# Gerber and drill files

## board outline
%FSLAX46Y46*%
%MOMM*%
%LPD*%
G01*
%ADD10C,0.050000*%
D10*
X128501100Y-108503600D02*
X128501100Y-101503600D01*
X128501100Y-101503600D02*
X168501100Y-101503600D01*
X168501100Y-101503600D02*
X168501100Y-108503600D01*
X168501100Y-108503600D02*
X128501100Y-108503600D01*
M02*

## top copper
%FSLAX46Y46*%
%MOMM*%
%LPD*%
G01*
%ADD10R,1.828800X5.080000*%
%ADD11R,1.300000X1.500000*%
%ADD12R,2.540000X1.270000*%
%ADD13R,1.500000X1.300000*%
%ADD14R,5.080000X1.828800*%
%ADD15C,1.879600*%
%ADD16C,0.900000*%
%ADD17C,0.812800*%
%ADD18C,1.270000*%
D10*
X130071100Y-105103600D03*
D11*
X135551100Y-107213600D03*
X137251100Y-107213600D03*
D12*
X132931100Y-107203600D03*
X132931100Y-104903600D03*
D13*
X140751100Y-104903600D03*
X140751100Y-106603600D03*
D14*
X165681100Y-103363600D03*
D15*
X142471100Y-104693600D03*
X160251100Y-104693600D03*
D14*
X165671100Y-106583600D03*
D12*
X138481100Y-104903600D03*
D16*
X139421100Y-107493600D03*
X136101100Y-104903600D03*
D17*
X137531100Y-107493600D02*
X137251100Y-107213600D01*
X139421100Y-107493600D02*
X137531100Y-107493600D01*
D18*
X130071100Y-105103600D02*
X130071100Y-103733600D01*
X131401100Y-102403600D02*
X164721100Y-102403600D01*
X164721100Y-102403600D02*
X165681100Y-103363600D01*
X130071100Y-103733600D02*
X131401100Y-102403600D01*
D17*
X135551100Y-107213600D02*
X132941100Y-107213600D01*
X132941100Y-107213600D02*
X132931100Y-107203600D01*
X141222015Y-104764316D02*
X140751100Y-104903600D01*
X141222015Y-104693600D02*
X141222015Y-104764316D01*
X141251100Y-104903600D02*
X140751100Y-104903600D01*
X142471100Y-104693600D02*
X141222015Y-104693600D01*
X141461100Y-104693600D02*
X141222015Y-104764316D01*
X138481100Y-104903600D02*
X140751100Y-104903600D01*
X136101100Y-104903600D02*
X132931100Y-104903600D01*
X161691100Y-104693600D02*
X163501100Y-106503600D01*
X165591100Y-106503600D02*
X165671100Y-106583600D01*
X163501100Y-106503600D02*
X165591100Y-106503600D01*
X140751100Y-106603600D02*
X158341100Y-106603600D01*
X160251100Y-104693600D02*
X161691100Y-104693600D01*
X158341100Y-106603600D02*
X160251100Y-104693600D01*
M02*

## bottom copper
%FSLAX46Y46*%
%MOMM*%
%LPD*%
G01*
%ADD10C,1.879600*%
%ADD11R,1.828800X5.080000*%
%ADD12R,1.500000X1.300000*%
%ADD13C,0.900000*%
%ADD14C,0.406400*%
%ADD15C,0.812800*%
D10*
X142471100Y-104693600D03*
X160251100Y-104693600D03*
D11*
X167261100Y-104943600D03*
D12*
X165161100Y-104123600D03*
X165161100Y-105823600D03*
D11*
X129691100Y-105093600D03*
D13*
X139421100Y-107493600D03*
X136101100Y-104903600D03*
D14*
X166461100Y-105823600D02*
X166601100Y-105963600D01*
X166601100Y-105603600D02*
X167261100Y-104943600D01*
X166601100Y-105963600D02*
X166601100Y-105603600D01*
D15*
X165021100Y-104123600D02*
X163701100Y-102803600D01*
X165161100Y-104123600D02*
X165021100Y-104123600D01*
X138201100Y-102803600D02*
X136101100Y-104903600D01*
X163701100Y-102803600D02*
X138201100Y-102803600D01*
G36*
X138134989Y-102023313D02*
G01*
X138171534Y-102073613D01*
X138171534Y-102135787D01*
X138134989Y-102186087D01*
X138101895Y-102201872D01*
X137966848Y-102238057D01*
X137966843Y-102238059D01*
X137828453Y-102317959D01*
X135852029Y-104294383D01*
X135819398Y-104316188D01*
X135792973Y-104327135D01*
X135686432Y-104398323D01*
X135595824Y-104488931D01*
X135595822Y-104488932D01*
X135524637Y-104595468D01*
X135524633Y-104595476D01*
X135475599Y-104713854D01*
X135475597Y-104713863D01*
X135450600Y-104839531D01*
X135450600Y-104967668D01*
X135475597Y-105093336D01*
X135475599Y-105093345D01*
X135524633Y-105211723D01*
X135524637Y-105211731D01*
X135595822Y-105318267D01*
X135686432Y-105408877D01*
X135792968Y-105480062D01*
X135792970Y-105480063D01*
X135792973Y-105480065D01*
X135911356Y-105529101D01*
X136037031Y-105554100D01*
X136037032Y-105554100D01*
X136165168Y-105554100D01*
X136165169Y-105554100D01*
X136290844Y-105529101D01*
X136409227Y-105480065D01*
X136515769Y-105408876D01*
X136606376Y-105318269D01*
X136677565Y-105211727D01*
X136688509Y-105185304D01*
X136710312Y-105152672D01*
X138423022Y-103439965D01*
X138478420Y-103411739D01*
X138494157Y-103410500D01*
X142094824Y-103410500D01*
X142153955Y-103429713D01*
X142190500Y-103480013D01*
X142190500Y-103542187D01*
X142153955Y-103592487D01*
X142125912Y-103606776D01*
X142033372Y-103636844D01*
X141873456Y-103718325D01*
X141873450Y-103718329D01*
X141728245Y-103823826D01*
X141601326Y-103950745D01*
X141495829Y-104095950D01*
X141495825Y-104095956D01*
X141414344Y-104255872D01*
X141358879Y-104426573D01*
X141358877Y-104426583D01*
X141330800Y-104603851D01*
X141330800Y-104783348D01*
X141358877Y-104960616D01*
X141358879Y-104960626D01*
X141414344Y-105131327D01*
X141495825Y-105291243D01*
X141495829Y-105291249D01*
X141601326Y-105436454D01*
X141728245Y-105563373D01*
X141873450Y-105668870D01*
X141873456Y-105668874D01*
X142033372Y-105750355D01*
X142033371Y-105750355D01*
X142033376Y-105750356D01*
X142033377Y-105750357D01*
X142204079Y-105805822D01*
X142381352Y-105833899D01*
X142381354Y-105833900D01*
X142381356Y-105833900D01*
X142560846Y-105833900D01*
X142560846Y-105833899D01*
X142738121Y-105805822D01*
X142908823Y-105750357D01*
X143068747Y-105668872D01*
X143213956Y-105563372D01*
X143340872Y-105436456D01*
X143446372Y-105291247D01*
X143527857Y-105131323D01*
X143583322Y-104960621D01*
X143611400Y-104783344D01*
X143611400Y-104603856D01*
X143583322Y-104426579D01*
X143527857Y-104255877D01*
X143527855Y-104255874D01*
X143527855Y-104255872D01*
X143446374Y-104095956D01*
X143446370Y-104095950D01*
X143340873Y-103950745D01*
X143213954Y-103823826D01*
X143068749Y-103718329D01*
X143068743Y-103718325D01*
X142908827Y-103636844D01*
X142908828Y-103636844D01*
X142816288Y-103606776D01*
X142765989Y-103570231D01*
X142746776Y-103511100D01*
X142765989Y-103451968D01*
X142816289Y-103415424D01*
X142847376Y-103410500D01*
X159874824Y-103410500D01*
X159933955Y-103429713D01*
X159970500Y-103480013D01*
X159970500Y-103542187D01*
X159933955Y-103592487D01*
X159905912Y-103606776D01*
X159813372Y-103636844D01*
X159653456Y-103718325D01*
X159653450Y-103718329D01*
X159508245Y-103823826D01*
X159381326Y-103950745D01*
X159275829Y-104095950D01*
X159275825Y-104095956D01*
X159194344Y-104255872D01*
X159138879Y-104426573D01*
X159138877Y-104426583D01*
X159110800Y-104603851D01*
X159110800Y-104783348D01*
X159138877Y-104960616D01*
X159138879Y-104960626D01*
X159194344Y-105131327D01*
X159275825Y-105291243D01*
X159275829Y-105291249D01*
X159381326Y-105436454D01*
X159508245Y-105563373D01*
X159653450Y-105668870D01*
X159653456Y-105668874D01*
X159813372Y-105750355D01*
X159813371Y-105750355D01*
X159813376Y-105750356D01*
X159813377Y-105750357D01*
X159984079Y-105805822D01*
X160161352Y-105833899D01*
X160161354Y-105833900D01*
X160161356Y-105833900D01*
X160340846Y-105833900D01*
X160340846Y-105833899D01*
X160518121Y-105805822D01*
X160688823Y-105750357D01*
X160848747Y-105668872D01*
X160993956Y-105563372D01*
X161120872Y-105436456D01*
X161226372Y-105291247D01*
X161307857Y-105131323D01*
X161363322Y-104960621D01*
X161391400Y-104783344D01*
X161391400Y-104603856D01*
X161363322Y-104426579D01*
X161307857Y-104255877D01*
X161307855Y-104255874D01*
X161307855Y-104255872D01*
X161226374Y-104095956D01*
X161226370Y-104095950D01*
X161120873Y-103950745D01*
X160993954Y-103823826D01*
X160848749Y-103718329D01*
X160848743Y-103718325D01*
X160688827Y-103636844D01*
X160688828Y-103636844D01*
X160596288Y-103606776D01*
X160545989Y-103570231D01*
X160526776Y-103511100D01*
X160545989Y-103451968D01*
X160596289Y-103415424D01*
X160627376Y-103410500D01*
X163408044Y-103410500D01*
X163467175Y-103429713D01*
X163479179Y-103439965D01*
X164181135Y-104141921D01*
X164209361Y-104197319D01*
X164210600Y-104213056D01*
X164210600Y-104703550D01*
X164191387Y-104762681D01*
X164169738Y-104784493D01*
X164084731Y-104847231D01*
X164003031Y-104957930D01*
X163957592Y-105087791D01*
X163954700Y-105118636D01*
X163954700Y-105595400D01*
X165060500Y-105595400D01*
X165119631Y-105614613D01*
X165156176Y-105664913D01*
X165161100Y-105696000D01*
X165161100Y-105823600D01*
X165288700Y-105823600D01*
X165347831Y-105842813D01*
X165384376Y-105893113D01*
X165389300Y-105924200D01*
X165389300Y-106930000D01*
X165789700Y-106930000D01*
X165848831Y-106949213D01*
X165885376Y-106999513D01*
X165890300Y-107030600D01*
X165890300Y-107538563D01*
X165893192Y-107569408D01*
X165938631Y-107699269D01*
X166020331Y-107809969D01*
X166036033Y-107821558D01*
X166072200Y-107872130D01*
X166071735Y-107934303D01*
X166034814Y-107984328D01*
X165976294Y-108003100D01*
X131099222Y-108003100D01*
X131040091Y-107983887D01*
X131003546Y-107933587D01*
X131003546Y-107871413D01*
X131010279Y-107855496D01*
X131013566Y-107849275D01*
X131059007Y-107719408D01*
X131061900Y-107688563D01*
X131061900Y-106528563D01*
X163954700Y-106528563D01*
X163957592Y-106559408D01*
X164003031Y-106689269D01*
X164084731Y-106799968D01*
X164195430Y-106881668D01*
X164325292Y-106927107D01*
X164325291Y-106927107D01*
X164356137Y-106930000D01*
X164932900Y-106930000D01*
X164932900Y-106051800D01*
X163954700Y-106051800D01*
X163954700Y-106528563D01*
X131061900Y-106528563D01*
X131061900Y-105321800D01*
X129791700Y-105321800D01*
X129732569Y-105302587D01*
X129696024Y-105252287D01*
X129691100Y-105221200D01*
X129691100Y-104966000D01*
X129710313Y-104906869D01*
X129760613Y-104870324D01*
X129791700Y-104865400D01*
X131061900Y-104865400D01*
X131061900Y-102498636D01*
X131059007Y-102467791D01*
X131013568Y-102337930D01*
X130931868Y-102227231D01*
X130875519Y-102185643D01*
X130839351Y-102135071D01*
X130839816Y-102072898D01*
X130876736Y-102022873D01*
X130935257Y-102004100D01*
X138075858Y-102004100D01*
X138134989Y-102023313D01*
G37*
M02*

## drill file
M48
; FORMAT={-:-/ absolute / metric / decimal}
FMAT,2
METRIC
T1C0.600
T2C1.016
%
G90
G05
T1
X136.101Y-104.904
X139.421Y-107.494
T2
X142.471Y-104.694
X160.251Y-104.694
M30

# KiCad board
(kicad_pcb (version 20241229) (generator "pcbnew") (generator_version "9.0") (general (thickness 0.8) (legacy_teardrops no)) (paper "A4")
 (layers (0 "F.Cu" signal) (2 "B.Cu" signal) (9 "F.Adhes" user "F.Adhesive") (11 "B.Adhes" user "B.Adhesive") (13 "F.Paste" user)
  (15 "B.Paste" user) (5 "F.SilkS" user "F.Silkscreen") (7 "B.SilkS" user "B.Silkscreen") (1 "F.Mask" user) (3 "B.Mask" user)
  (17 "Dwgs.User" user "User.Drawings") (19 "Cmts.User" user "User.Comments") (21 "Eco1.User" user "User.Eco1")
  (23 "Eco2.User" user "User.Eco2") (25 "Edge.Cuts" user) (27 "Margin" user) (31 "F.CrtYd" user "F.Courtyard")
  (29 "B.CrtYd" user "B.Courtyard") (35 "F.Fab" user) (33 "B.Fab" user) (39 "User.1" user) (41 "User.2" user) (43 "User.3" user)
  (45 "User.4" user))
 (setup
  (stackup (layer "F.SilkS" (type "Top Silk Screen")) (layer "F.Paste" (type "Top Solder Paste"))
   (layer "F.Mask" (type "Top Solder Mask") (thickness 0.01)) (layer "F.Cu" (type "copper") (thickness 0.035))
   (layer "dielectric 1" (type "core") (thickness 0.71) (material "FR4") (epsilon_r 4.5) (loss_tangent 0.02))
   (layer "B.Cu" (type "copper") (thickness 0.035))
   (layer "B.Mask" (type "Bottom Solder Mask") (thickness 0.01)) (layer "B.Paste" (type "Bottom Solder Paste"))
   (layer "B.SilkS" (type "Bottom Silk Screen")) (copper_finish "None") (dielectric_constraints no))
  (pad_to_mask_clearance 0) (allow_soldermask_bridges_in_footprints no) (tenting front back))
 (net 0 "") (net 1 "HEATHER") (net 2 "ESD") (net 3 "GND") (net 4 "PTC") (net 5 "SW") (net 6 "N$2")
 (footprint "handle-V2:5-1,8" (layer "F.Cu") (at 130.0711 105.1036 180)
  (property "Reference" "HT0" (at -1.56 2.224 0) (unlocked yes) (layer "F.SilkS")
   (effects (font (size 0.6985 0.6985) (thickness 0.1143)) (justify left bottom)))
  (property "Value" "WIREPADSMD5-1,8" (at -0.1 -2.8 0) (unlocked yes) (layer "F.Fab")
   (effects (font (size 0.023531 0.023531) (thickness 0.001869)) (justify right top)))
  (pad "1" smd rect (at 0 0 180) (size 1.8288 5.08) (layers "F.Cu" "F.Mask" "F.Paste") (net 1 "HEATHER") (solder_mask_margin 0)
   (solder_paste_margin 0) (thermal_bridge_angle 0)))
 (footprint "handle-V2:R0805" (layer "F.Cu") (at 136.4011 107.2136)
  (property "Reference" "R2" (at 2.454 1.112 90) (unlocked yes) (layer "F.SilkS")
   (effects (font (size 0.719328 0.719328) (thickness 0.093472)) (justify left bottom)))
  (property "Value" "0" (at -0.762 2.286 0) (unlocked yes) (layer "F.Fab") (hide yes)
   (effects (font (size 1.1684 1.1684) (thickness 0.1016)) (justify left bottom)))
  (pad "1" smd rect (at -0.85 0) (size 1.3 1.5) (layers "F.Cu" "F.Mask" "F.Paste") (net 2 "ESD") (solder_mask_margin 0)
   (solder_paste_margin 0) (thermal_bridge_angle 0))
  (pad "2" smd rect (at 0.85 0) (size 1.3 1.5) (layers "F.Cu" "F.Mask" "F.Paste") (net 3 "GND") (solder_mask_margin 0)
   (solder_paste_margin 0) (thermal_bridge_angle 0)))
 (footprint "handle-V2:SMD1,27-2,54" (layer "F.Cu") (at 132.9311 107.2036 -90)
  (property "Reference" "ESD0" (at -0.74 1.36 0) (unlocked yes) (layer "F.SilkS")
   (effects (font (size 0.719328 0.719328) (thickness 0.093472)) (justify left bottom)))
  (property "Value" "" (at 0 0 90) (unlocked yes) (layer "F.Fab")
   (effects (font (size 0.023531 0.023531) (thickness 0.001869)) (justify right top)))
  (pad "1" smd rect (at 0 0 270) (size 1.27 2.54) (layers "F.Cu" "F.Mask" "F.Paste") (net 2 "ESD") (solder_mask_margin 0)
   (solder_paste_margin 0) (thermal_bridge_angle 0)))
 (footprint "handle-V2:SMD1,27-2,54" (layer "F.Cu") (at 132.9311 104.9036 -90)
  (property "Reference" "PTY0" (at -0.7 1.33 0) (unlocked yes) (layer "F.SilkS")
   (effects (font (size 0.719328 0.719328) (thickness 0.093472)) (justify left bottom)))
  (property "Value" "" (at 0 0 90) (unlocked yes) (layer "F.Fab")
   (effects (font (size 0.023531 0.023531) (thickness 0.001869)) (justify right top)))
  (pad "1" smd rect (at 0 0 270) (size 1.27 2.54) (layers "F.Cu" "F.Mask" "F.Paste") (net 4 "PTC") (solder_mask_margin 0)
   (solder_paste_margin 0) (thermal_bridge_angle 0)))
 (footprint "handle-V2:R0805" (layer "F.Cu") (at 140.7511 105.7536 -90)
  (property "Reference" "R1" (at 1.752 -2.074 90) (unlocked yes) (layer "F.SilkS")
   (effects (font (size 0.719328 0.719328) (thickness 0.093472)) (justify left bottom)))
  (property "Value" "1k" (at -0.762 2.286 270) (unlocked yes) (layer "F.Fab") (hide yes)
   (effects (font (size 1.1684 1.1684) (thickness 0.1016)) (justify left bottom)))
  (pad "1" smd rect (at -0.85 0 270) (size 1.3 1.5) (layers "F.Cu" "F.Mask" "F.Paste") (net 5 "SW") (solder_mask_margin 0)
   (solder_paste_margin 0) (thermal_bridge_angle 0))
  (pad "2" smd rect (at 0.85 0 270) (size 1.3 1.5) (layers "F.Cu" "F.Mask" "F.Paste") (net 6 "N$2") (solder_mask_margin 0)
   (solder_paste_margin 0) (thermal_bridge_angle 0)))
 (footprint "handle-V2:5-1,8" (layer "F.Cu") (at 165.6811 103.3636 90)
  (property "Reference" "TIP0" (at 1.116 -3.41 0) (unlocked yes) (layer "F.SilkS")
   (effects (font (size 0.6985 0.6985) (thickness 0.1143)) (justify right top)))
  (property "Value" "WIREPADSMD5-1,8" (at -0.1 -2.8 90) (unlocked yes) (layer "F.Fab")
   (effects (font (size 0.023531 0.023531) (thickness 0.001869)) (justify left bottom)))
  (pad "1" smd rect (at 0 0 90) (size 1.8288 5.08) (layers "F.Cu" "F.Mask" "F.Paste") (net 1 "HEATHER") (solder_mask_margin 0)
   (solder_paste_margin 0) (thermal_bridge_angle 0)))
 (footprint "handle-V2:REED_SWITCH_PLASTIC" (layer "F.Cu") (at 151.3611 104.6936)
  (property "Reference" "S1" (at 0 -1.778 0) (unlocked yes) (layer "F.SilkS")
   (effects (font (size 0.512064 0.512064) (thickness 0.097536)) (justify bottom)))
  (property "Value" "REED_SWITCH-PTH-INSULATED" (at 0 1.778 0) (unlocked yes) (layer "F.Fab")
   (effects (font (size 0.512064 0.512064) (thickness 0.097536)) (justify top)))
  (pad "P$1" thru_hole circle (at -8.89 0) (size 1.8796 1.8796) (drill 1.016) (layers "*.Cu" "*.Mask") (remove_unused_layers no)
   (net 5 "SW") (solder_mask_margin 0) (thermal_bridge_angle 0))
  (pad "P$2" thru_hole circle (at 8.89 0) (size 1.8796 1.8796) (drill 1.016) (layers "*.Cu" "*.Mask") (remove_unused_layers no)
   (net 6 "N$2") (solder_mask_margin 0) (thermal_bridge_angle 0)))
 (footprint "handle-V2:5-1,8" (layer "F.Cu") (at 165.6711 106.5836 90)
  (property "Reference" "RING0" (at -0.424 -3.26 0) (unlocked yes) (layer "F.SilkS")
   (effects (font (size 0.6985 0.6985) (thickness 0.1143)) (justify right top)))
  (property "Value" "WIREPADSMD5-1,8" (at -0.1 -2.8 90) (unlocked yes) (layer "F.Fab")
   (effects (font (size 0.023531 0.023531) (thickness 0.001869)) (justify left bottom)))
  (pad "1" smd rect (at 0 0 90) (size 1.8288 5.08) (layers "F.Cu" "F.Mask" "F.Paste") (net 6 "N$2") (solder_mask_margin 0)
   (solder_paste_margin 0) (thermal_bridge_angle 0)))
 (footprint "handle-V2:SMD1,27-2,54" (layer "F.Cu") (at 138.4811 104.9036 -90)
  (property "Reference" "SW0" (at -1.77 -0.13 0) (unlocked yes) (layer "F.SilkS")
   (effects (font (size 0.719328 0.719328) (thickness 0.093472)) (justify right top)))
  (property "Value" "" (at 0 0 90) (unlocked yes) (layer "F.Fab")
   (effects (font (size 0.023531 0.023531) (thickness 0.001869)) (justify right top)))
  (pad "1" smd rect (at 0 0 270) (size 1.27 2.54) (layers "F.Cu" "F.Mask" "F.Paste") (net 5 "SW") (solder_mask_margin 0)
   (solder_paste_margin 0) (thermal_bridge_angle 0)))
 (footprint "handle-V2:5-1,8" (layer "B.Cu") (at 167.2611 104.9436)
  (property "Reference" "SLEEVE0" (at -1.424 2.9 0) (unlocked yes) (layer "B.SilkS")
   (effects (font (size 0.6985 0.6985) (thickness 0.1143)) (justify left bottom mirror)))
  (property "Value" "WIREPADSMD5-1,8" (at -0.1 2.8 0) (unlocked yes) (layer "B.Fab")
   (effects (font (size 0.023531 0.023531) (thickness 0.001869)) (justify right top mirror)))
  (pad "1" smd rect (at 0 0) (size 1.8288 5.08) (layers "B.Cu" "B.Mask" "B.Paste") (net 3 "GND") (solder_mask_margin 0)
   (solder_paste_margin 0) (thermal_bridge_angle 0)))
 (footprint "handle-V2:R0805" (layer "B.Cu") (at 165.1611 104.9736 -90)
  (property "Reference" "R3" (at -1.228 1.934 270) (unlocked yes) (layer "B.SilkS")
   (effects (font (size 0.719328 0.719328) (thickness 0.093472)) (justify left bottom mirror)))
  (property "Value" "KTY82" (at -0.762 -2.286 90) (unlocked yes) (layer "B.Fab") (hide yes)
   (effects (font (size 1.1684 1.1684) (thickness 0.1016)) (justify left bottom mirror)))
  (pad "1" smd rect (at -0.85 0 270) (size 1.3 1.5) (layers "B.Cu" "B.Mask" "B.Paste") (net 4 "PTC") (solder_mask_margin 0)
   (solder_paste_margin 0) (thermal_bridge_angle 0))
  (pad "2" smd rect (at 0.85 0 270) (size 1.3 1.5) (layers "B.Cu" "B.Mask" "B.Paste") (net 3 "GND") (solder_mask_margin 0)
   (solder_paste_margin 0) (thermal_bridge_angle 0)))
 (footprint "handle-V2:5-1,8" (layer "B.Cu") (at 129.6911 105.0936)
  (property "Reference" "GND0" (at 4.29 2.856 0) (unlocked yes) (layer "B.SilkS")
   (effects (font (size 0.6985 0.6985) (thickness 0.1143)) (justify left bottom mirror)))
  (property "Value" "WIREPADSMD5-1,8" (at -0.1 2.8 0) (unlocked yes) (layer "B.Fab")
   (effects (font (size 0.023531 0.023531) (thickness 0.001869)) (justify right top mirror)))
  (pad "1" smd rect (at 0 0) (size 1.8288 5.08) (layers "B.Cu" "B.Mask" "B.Paste") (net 3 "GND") (solder_mask_margin 0)
   (solder_paste_margin 0) (thermal_bridge_angle 0)))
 (gr_line (start 128.5011 108.5036) (end 128.5011 101.5036) (stroke (width 0.05) (type solid)) (layer "Edge.Cuts"))
 (gr_line (start 128.5011 101.5036) (end 168.5011 101.5036) (stroke (width 0.05) (type solid)) (layer "Edge.Cuts"))
 (gr_line (start 168.5011 101.5036) (end 168.5011 108.5036) (stroke (width 0.05) (type solid)) (layer "Edge.Cuts"))
 (gr_line (start 168.5011 108.5036) (end 128.5011 108.5036) (stroke (width 0.05) (type solid)) (layer "Edge.Cuts"))
 (segment (start 137.5311 107.4936) (end 137.2511 107.2136) (width 0.8128) (layer "F.Cu") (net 3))
 (segment (start 139.4211 107.4936) (end 137.5311 107.4936) (width 0.8128) (layer "F.Cu") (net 3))
 (via (at 139.4211 107.4936) (size 0.9) (drill 0.6) (layers "F.Cu" "B.Cu") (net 3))
 (segment (start 166.4611 105.8236) (end 166.6011 105.9636) (width 0.4064) (layer "B.Cu") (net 3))
 (segment (start 166.6011 105.6036) (end 167.2611 104.9436) (width 0.4064) (layer "B.Cu") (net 3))
 (segment (start 166.6011 105.9636) (end 166.6011 105.6036) (width 0.4064) (layer "B.Cu") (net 3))
 (segment (start 130.0711 105.1036) (end 130.0711 103.7336) (width 1.27) (layer "F.Cu") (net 1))
 (segment (start 131.4011 102.4036) (end 164.7211 102.4036) (width 1.27) (layer "F.Cu") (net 1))
 (segment (start 164.7211 102.4036) (end 165.6811 103.3636) (width 1.27) (layer "F.Cu") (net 1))
 (segment (start 130.0711 103.7336) (end 131.4011 102.4036) (width 1.27) (layer "F.Cu") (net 1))
 (segment (start 135.5511 107.2136) (end 132.9411 107.2136) (width 0.8128) (layer "F.Cu") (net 2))
 (segment (start 132.9411 107.2136) (end 132.9311 107.2036) (width 0.8128) (layer "F.Cu") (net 2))
 (segment (start 141.222015 104.764316) (end 140.7511 104.9036) (width 0.8128) (layer "F.Cu") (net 5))
 (segment (start 141.222015 104.6936) (end 141.222015 104.764316) (width 0.8128) (layer "F.Cu") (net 5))
 (segment (start 141.2511 104.9036) (end 140.7511 104.9036) (width 0.8128) (layer "F.Cu") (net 5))
 (segment (start 142.4711 104.6936) (end 141.222015 104.6936) (width 0.8128) (layer "F.Cu") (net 5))
 (segment (start 141.4611 104.6936) (end 141.222015 104.764316) (width 0.8128) (layer "F.Cu") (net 5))
 (segment (start 138.4811 104.9036) (end 140.7511 104.9036) (width 0.8128) (layer "F.Cu") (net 5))
 (segment (start 136.1011 104.9036) (end 132.9311 104.9036) (width 0.8128) (layer "F.Cu") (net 4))
 (via (at 136.1011 104.9036) (size 0.9) (drill 0.6) (layers "F.Cu" "B.Cu") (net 4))
 (segment (start 165.0211 104.1236) (end 163.7011 102.8036) (width 0.8128) (layer "B.Cu") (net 4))
 (segment (start 165.1611 104.1236) (end 165.0211 104.1236) (width 0.8128) (layer "B.Cu") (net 4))
 (segment (start 138.2011 102.8036) (end 136.1011 104.9036) (width 0.8128) (layer "B.Cu") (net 4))
 (segment (start 163.7011 102.8036) (end 138.2011 102.8036) (width 0.8128) (layer "B.Cu") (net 4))
 (segment (start 161.6911 104.6936) (end 163.5011 106.5036) (width 0.8128) (layer "F.Cu") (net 6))
 (segment (start 165.5911 106.5036) (end 165.6711 106.5836) (width 0.8128) (layer "F.Cu") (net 6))
 (segment (start 163.5011 106.5036) (end 165.5911 106.5036) (width 0.8128) (layer "F.Cu") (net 6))
 (segment (start 140.7511 106.6036) (end 158.3411 106.6036) (width 0.8128) (layer "F.Cu") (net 6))
 (segment (start 160.2511 104.6936) (end 161.6911 104.6936) (width 0.8128) (layer "F.Cu") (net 6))
 (segment (start 158.3411 106.6036) (end 160.2511 104.6936) (width 0.8128) (layer "F.Cu") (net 6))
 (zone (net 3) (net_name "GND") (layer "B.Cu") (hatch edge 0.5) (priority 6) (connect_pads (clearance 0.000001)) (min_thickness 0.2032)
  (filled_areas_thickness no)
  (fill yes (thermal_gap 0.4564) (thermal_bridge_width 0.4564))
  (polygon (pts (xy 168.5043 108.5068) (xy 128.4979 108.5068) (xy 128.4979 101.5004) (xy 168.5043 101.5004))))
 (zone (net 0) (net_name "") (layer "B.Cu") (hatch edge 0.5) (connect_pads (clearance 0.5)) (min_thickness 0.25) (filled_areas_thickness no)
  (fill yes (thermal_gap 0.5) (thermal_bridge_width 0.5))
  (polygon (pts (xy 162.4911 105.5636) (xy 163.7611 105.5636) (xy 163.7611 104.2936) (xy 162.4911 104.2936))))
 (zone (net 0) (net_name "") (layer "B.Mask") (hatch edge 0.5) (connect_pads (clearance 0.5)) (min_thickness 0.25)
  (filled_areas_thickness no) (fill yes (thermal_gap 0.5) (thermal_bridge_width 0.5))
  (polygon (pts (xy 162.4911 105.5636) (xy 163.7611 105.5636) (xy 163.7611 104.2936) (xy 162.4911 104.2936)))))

